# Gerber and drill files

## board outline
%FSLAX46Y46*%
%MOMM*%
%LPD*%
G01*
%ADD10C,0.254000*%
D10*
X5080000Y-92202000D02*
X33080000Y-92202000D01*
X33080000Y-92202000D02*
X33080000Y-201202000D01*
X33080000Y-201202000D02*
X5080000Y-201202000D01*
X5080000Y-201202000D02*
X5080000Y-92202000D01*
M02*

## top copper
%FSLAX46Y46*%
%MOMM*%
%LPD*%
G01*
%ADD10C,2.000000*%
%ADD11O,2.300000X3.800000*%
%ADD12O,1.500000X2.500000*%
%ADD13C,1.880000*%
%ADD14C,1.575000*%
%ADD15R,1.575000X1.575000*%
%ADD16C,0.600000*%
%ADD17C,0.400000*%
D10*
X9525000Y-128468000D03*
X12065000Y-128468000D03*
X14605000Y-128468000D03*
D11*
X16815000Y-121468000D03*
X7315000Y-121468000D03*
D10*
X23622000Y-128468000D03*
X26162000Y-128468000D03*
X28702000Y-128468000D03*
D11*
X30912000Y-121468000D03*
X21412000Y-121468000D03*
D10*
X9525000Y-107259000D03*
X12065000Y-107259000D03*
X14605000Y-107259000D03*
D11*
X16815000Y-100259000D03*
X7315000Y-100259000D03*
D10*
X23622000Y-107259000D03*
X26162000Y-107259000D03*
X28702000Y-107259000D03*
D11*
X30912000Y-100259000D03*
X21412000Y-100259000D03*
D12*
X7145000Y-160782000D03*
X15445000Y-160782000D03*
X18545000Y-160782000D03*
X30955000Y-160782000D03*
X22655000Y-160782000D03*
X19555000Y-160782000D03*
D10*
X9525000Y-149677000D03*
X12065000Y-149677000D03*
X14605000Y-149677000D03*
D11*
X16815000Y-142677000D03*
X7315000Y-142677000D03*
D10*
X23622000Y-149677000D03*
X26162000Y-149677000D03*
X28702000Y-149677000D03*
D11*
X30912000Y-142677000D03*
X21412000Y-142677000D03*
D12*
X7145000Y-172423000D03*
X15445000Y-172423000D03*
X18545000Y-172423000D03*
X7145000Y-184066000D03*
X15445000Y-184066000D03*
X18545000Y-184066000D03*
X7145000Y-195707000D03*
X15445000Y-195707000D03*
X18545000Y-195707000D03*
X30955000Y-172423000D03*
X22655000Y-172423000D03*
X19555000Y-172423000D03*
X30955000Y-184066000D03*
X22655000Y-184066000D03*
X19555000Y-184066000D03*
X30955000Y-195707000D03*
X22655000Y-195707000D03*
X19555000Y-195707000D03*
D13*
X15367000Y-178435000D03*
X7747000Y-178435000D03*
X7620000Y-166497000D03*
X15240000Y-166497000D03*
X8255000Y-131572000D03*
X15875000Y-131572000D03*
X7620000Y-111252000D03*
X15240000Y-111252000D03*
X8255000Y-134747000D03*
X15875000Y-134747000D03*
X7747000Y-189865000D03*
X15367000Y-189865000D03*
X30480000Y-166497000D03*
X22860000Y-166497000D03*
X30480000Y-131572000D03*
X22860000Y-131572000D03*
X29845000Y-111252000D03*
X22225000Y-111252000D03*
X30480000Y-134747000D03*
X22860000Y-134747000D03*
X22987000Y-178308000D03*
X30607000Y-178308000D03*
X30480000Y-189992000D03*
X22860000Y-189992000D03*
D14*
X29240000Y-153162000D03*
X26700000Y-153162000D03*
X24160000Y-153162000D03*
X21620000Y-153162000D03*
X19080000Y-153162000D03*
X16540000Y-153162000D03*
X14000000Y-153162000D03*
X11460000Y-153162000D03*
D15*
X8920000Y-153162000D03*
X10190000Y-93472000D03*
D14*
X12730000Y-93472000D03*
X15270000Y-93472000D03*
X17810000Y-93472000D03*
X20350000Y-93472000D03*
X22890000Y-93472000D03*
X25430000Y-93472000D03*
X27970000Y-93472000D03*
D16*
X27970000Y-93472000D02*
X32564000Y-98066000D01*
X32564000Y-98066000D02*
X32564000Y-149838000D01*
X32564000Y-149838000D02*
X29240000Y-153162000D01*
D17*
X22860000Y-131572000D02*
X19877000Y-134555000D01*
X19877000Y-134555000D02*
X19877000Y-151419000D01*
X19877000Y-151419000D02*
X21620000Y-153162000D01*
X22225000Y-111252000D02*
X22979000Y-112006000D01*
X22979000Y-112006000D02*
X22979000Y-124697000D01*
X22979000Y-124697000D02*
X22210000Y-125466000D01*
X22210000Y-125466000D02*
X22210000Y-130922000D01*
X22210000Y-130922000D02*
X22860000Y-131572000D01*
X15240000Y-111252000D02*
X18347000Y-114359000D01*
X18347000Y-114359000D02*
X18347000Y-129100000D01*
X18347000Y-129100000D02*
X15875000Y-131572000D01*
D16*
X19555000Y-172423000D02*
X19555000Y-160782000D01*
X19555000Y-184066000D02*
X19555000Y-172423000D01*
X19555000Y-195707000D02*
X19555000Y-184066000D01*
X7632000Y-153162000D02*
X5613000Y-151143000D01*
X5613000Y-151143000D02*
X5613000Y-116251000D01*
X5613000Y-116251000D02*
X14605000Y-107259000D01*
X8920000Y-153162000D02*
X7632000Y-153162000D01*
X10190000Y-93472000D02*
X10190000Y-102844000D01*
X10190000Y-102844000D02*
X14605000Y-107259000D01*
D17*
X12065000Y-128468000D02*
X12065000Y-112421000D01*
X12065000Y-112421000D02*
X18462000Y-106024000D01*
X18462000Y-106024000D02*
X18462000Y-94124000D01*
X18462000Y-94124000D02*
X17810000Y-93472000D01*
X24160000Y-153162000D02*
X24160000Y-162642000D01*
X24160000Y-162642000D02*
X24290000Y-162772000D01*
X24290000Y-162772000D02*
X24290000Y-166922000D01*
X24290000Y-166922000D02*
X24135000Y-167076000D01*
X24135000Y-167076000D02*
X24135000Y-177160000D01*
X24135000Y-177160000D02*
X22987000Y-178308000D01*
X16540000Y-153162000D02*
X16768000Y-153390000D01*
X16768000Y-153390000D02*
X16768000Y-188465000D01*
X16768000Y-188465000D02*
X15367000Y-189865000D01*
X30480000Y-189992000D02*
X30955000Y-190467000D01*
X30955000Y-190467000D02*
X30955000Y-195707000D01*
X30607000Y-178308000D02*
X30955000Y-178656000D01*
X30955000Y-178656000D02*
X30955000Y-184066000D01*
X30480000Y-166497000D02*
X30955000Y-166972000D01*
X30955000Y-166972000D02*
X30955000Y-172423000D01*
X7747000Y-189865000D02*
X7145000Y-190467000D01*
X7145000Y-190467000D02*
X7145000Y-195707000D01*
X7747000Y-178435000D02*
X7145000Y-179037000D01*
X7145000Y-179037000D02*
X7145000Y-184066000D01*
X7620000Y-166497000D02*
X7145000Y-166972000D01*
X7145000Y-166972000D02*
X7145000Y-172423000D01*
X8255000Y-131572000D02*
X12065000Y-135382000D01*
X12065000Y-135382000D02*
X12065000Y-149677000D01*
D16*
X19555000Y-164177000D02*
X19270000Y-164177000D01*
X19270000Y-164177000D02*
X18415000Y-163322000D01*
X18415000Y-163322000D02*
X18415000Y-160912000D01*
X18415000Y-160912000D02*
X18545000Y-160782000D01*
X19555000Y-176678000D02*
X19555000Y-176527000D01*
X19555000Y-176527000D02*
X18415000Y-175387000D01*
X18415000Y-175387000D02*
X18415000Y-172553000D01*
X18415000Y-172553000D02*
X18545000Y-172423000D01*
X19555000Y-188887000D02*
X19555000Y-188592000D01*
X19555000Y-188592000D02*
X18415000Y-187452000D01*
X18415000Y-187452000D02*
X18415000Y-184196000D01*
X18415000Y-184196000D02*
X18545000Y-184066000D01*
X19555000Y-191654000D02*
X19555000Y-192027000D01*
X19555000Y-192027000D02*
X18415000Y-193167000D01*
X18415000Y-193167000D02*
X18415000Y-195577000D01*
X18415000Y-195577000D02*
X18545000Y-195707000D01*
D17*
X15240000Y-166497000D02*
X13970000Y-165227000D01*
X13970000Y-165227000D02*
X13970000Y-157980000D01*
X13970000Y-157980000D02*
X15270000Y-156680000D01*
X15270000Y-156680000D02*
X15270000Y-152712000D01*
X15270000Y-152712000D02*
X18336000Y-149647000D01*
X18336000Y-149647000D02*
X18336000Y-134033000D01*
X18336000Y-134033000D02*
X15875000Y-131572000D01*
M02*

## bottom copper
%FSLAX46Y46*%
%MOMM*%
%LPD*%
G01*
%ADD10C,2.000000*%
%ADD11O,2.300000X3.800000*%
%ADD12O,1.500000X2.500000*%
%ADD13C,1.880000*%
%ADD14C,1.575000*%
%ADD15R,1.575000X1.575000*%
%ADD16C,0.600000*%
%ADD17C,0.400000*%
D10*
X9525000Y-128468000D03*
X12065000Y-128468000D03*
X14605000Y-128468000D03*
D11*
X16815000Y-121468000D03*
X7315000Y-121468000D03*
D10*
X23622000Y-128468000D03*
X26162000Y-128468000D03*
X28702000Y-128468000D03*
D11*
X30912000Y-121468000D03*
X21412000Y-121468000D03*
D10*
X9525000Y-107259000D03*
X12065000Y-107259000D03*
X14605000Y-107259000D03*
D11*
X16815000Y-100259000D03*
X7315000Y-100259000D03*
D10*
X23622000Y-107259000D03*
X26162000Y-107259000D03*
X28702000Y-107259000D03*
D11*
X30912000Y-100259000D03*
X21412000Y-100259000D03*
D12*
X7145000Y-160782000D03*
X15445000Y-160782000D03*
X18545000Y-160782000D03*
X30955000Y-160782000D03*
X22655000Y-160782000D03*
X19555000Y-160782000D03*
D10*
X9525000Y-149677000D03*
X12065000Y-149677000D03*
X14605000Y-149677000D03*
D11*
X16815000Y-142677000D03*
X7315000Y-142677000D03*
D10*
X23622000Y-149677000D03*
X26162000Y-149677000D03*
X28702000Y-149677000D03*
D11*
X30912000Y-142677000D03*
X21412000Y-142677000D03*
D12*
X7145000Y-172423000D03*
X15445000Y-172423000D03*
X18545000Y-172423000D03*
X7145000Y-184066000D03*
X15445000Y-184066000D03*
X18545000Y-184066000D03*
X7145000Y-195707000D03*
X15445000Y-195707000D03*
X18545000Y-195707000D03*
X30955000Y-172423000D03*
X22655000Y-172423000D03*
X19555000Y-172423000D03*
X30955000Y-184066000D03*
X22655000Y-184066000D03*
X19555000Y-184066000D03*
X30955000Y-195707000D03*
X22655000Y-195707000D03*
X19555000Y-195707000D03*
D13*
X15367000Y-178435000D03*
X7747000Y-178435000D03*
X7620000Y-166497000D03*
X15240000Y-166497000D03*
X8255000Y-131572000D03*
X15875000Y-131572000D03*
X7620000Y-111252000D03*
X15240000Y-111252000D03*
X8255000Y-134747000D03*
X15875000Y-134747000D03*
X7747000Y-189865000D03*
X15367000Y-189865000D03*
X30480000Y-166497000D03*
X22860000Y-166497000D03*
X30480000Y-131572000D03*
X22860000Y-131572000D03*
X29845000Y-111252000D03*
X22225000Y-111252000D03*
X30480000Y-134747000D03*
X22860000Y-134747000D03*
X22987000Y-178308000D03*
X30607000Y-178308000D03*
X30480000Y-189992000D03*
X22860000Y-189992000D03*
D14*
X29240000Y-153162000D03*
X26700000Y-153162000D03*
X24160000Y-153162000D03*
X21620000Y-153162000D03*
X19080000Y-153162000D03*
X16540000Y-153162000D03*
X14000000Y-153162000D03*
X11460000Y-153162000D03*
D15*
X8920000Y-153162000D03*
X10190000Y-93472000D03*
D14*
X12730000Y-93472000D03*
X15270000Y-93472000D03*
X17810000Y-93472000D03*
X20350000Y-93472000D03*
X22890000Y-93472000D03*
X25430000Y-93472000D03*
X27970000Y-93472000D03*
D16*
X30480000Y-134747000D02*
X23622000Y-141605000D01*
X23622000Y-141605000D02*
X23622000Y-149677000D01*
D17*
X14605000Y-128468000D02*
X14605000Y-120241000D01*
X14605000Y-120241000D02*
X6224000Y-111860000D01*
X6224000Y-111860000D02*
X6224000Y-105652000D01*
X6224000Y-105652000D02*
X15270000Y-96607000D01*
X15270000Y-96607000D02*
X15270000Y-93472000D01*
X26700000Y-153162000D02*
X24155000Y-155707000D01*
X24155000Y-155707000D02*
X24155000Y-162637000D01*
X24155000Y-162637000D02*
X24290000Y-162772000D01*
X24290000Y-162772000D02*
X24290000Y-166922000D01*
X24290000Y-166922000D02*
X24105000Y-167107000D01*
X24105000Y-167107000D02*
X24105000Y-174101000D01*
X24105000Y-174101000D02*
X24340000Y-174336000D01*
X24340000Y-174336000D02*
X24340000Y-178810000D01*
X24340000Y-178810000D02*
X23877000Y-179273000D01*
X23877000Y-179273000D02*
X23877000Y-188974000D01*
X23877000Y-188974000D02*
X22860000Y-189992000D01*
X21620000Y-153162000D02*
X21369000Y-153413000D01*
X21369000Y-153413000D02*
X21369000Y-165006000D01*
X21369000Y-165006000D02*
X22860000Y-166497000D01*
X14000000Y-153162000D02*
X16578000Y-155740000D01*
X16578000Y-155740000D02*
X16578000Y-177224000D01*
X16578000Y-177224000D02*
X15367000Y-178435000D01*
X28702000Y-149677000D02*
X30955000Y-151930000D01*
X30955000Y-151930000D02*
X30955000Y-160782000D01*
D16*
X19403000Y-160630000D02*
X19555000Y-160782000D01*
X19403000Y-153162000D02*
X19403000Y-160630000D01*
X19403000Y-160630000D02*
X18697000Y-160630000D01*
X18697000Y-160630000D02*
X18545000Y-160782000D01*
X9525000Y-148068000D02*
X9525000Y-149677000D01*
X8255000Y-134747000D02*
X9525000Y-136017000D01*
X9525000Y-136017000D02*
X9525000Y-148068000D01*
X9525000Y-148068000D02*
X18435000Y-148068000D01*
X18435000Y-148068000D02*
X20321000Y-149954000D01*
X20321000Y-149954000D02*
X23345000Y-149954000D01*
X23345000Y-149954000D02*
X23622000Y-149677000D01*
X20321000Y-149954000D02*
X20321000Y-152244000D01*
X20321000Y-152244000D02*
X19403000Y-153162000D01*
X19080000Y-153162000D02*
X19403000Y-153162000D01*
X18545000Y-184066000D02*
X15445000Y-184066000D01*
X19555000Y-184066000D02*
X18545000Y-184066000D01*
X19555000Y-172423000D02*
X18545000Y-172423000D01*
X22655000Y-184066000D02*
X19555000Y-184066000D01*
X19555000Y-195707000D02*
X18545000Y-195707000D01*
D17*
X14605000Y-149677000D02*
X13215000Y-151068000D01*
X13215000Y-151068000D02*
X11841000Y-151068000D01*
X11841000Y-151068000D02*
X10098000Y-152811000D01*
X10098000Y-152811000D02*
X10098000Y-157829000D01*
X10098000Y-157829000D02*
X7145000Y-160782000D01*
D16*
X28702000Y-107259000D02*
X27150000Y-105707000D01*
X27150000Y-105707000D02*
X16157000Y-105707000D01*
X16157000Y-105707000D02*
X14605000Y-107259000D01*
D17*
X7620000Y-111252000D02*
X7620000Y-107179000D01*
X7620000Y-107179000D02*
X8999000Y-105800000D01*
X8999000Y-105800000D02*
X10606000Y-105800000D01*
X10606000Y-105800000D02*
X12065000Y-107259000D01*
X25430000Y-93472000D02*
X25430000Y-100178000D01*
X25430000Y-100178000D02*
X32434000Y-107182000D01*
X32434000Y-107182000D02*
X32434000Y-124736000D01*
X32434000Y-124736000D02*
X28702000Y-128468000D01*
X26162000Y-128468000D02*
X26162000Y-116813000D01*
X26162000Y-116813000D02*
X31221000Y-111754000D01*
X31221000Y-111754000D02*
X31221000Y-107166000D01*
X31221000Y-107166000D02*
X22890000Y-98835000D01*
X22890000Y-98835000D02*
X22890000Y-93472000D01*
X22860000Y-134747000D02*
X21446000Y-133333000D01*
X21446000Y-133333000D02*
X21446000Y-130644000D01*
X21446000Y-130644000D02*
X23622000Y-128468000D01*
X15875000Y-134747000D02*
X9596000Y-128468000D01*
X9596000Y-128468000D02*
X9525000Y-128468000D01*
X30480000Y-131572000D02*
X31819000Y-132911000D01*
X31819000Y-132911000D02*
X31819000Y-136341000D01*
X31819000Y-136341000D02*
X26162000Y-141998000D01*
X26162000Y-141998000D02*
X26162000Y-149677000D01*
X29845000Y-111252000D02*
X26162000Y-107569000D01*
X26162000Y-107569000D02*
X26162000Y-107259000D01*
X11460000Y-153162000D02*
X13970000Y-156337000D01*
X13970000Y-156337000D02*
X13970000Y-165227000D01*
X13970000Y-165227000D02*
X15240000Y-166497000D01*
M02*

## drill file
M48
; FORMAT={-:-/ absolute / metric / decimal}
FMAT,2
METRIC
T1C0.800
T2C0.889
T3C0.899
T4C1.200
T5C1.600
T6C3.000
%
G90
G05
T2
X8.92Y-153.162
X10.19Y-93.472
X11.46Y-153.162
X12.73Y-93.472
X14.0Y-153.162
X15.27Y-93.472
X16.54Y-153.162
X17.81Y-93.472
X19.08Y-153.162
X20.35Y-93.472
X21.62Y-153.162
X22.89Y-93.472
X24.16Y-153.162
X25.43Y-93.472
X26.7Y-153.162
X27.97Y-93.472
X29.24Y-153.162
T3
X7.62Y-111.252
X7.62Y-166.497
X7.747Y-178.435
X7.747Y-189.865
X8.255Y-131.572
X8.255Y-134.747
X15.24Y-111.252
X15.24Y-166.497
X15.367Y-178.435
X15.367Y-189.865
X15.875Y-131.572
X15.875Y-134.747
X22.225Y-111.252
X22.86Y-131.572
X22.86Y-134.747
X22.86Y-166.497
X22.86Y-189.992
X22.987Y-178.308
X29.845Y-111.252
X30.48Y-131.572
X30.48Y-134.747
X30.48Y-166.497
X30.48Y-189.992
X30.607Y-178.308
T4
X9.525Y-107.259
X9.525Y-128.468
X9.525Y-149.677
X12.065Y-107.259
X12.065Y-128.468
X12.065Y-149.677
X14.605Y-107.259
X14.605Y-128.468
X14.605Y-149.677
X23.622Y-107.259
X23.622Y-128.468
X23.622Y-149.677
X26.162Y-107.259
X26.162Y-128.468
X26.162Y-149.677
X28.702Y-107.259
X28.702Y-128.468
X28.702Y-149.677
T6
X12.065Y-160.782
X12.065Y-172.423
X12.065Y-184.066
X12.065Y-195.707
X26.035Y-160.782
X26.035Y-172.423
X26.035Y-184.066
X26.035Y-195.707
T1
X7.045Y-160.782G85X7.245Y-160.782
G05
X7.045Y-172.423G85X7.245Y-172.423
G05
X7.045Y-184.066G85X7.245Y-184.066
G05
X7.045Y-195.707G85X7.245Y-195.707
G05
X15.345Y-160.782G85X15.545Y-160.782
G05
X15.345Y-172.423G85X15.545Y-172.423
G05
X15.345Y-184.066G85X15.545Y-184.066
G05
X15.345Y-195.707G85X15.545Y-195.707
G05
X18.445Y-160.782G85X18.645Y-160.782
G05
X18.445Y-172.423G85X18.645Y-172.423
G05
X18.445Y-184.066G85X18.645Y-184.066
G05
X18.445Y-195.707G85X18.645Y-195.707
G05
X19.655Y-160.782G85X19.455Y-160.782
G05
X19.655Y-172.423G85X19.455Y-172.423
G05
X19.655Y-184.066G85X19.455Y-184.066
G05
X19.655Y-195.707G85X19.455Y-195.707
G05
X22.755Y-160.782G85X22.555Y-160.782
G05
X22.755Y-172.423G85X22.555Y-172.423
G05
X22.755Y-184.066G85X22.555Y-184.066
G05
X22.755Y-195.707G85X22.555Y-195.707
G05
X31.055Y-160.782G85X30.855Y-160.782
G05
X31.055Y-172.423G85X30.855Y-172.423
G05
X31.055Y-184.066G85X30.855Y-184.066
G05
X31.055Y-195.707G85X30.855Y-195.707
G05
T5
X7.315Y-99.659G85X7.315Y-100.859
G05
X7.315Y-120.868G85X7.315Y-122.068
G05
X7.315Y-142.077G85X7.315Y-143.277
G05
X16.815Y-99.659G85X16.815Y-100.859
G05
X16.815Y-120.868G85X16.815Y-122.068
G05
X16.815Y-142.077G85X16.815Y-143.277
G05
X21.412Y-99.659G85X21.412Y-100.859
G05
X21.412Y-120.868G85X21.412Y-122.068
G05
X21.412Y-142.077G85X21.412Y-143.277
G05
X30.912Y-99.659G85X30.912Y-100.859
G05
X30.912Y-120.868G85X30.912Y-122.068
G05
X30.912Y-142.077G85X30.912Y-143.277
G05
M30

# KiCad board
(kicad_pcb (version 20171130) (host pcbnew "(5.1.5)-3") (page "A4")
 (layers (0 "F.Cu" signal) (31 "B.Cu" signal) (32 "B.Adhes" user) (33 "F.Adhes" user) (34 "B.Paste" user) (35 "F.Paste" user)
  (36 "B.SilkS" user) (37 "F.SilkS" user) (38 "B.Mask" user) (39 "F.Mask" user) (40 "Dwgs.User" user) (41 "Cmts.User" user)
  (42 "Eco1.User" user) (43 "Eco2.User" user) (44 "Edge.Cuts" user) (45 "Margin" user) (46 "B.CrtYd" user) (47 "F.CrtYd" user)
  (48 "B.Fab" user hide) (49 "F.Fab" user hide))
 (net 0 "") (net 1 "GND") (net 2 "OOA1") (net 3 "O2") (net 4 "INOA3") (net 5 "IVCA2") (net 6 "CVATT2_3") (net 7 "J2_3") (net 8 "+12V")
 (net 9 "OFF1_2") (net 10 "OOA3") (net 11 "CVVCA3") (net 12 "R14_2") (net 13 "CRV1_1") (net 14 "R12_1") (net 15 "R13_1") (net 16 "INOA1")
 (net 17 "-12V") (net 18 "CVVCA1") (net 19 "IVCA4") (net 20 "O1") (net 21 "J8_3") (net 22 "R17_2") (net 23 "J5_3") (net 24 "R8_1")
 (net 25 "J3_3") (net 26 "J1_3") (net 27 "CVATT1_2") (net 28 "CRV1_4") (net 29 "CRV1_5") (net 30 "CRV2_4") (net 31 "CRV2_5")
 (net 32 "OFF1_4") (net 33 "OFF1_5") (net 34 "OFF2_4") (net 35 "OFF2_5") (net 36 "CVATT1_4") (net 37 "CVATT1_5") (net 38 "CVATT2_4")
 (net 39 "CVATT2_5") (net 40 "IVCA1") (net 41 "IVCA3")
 (segment (start 30.48 134.747) (end 23.622 141.605) (width 0.6) (layer "B.Cu") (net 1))
 (segment (start 23.622 141.605) (end 23.622 149.677) (width 0.6) (layer "B.Cu") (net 1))
 (segment (start 14.605 128.468) (end 14.605 120.241) (width 0.4) (layer "B.Cu") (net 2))
 (segment (start 14.605 120.241) (end 6.224 111.86) (width 0.4) (layer "B.Cu") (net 2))
 (segment (start 6.224 111.86) (end 6.224 105.652) (width 0.4) (layer "B.Cu") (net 2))
 (segment (start 6.224 105.652) (end 15.27 96.607) (width 0.4) (layer "B.Cu") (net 2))
 (segment (start 15.27 96.607) (end 15.27 93.472) (width 0.4) (layer "B.Cu") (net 2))
 (segment (start 26.7 153.162) (end 24.155 155.707) (width 0.4) (layer "B.Cu") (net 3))
 (segment (start 24.155 155.707) (end 24.155 162.637) (width 0.4) (layer "B.Cu") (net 3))
 (segment (start 24.155 162.637) (end 24.29 162.772) (width 0.4) (layer "B.Cu") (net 3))
 (segment (start 24.29 162.772) (end 24.29 166.922) (width 0.4) (layer "B.Cu") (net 3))
 (segment (start 24.29 166.922) (end 24.105 167.107) (width 0.4) (layer "B.Cu") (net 3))
 (segment (start 24.105 167.107) (end 24.105 174.101) (width 0.4) (layer "B.Cu") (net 3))
 (segment (start 24.105 174.101) (end 24.34 174.336) (width 0.4) (layer "B.Cu") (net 3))
 (segment (start 24.34 174.336) (end 24.34 178.81) (width 0.4) (layer "B.Cu") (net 3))
 (segment (start 24.34 178.81) (end 23.877 179.273) (width 0.4) (layer "B.Cu") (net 3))
 (segment (start 23.877 179.273) (end 23.877 188.974) (width 0.4) (layer "B.Cu") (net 3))
 (segment (start 23.877 188.974) (end 22.86 189.992) (width 0.4) (layer "B.Cu") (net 3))
 (segment (start 21.62 153.162) (end 21.369 153.413) (width 0.4) (layer "B.Cu") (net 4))
 (segment (start 21.369 153.413) (end 21.369 165.006) (width 0.4) (layer "B.Cu") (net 4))
 (segment (start 21.369 165.006) (end 22.86 166.497) (width 0.4) (layer "B.Cu") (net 4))
 (segment (start 14 153.162) (end 16.578 155.74) (width 0.4) (layer "B.Cu") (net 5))
 (segment (start 16.578 155.74) (end 16.578 177.224) (width 0.4) (layer "B.Cu") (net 5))
 (segment (start 16.578 177.224) (end 15.367 178.435) (width 0.4) (layer "B.Cu") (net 5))
 (segment (start 28.702 149.677) (end 30.955 151.93) (width 0.4) (layer "B.Cu") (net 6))
 (segment (start 30.955 151.93) (end 30.955 160.782) (width 0.4) (layer "B.Cu") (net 6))
 (segment (start 19.403 160.63) (end 19.555 160.782) (width 0.6) (layer "B.Cu") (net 1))
 (segment (start 19.403 153.162) (end 19.403 160.63) (width 0.6) (layer "B.Cu") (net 1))
 (segment (start 19.403 160.63) (end 18.697 160.63) (width 0.6) (layer "B.Cu") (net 1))
 (segment (start 18.697 160.63) (end 18.545 160.782) (width 0.6) (layer "B.Cu") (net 1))
 (segment (start 9.525 148.068) (end 9.525 149.677) (width 0.6) (layer "B.Cu") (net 1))
 (segment (start 8.255 134.747) (end 9.525 136.017) (width 0.6) (layer "B.Cu") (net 1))
 (segment (start 9.525 136.017) (end 9.525 148.068) (width 0.6) (layer "B.Cu") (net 1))
 (segment (start 9.525 148.068) (end 18.435 148.068) (width 0.6) (layer "B.Cu") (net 1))
 (segment (start 18.435 148.068) (end 20.321 149.954) (width 0.6) (layer "B.Cu") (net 1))
 (segment (start 20.321 149.954) (end 23.345 149.954) (width 0.6) (layer "B.Cu") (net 1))
 (segment (start 23.345 149.954) (end 23.622 149.677) (width 0.6) (layer "B.Cu") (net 1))
 (segment (start 20.321 149.954) (end 20.321 152.244) (width 0.6) (layer "B.Cu") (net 1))
 (segment (start 20.321 152.244) (end 19.403 153.162) (width 0.6) (layer "B.Cu") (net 1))
 (segment (start 19.08 153.162) (end 19.403 153.162) (width 0.6) (layer "B.Cu") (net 1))
 (segment (start 18.545 184.066) (end 15.445 184.066) (width 0.6) (layer "B.Cu") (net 1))
 (segment (start 19.555 184.066) (end 18.545 184.066) (width 0.6) (layer "B.Cu") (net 1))
 (segment (start 19.555 172.423) (end 18.545 172.423) (width 0.6) (layer "B.Cu") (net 1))
 (segment (start 22.655 184.066) (end 19.555 184.066) (width 0.6) (layer "B.Cu") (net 1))
 (segment (start 19.555 195.707) (end 18.545 195.707) (width 0.6) (layer "B.Cu") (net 1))
 (segment (start 14.605 149.677) (end 13.215 151.068) (width 0.4) (layer "B.Cu") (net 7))
 (segment (start 13.215 151.068) (end 11.841 151.068) (width 0.4) (layer "B.Cu") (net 7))
 (segment (start 11.841 151.068) (end 10.098 152.811) (width 0.4) (layer "B.Cu") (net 7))
 (segment (start 10.098 152.811) (end 10.098 157.829) (width 0.4) (layer "B.Cu") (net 7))
 (segment (start 10.098 157.829) (end 7.145 160.782) (width 0.4) (layer "B.Cu") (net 7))
 (segment (start 28.702 107.259) (end 27.15 105.707) (width 0.6) (layer "B.Cu") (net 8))
 (segment (start 27.15 105.707) (end 16.157 105.707) (width 0.6) (layer "B.Cu") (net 8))
 (segment (start 16.157 105.707) (end 14.605 107.259) (width 0.6) (layer "B.Cu") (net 8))
 (segment (start 7.62 111.252) (end 7.62 107.179) (width 0.4) (layer "B.Cu") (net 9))
 (segment (start 7.62 107.179) (end 8.999 105.8) (width 0.4) (layer "B.Cu") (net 9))
 (segment (start 8.999 105.8) (end 10.606 105.8) (width 0.4) (layer "B.Cu") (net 9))
 (segment (start 10.606 105.8) (end 12.065 107.259) (width 0.4) (layer "B.Cu") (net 9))
 (segment (start 25.43 93.472) (end 25.43 100.178) (width 0.4) (layer "B.Cu") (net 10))
 (segment (start 25.43 100.178) (end 32.434 107.182) (width 0.4) (layer "B.Cu") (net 10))
 (segment (start 32.434 107.182) (end 32.434 124.736) (width 0.4) (layer "B.Cu") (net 10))
 (segment (start 32.434 124.736) (end 28.702 128.468) (width 0.4) (layer "B.Cu") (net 10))
 (segment (start 26.162 128.468) (end 26.162 116.813) (width 0.4) (layer "B.Cu") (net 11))
 (segment (start 26.162 116.813) (end 31.221 111.754) (width 0.4) (layer "B.Cu") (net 11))
 (segment (start 31.221 111.754) (end 31.221 107.166) (width 0.4) (layer "B.Cu") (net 11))
 (segment (start 31.221 107.166) (end 22.89 98.835) (width 0.4) (layer "B.Cu") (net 11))
 (segment (start 22.89 98.835) (end 22.89 93.472) (width 0.4) (layer "B.Cu") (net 11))
 (segment (start 22.86 134.747) (end 21.446 133.333) (width 0.4) (layer "B.Cu") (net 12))
 (segment (start 21.446 133.333) (end 21.446 130.644) (width 0.4) (layer "B.Cu") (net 12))
 (segment (start 21.446 130.644) (end 23.622 128.468) (width 0.4) (layer "B.Cu") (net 12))
 (segment (start 15.875 134.747) (end 9.596 128.468) (width 0.4) (layer "B.Cu") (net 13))
 (segment (start 9.596 128.468) (end 9.525 128.468) (width 0.4) (layer "B.Cu") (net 13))
 (segment (start 30.48 131.572) (end 31.819 132.911) (width 0.4) (layer "B.Cu") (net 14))
 (segment (start 31.819 132.911) (end 31.819 136.341) (width 0.4) (layer "B.Cu") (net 14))
 (segment (start 31.819 136.341) (end 26.162 141.998) (width 0.4) (layer "B.Cu") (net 14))
 (segment (start 26.162 141.998) (end 26.162 149.677) (width 0.4) (layer "B.Cu") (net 14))
 (segment (start 29.845 111.252) (end 26.162 107.569) (width 0.4) (layer "B.Cu") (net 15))
 (segment (start 26.162 107.569) (end 26.162 107.259) (width 0.4) (layer "B.Cu") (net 15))
 (segment (start 11.46 153.162) (end 13.97 156.337) (width 0.4) (layer "B.Cu") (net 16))
 (segment (start 13.97 156.337) (end 13.97 165.227) (width 0.4) (layer "B.Cu") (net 16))
 (segment (start 13.97 165.227) (end 15.24 166.497) (width 0.4) (layer "B.Cu") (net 16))
 (gr_line (start 5.08 92.202) (end 33.08 92.202) (width 0.254) (layer "Edge.Cuts"))
 (gr_line (start 33.08 92.202) (end 33.08 201.202) (width 0.254) (layer "Edge.Cuts"))
 (gr_line (start 33.08 201.202) (end 5.08 201.202) (width 0.254) (layer "Edge.Cuts"))
 (gr_line (start 5.08 201.202) (end 5.08 92.202) (width 0.254) (layer "Edge.Cuts"))
 (segment (start 27.97 93.472) (end 32.564 98.066) (width 0.6) (layer "F.Cu") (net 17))
 (segment (start 32.564 98.066) (end 32.564 149.838) (width 0.6) (layer "F.Cu") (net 17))
 (segment (start 32.564 149.838) (end 29.24 153.162) (width 0.6) (layer "F.Cu") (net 17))
 (segment (start 22.86 131.572) (end 19.877 134.555) (width 0.4) (layer "F.Cu") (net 4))
 (segment (start 19.877 134.555) (end 19.877 151.419) (width 0.4) (layer "F.Cu") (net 4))
 (segment (start 19.877 151.419) (end 21.62 153.162) (width 0.4) (layer "F.Cu") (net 4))
 (segment (start 22.225 111.252) (end 22.979 112.006) (width 0.4) (layer "F.Cu") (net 4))
 (segment (start 22.979 112.006) (end 22.979 124.697) (width 0.4) (layer "F.Cu") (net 4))
 (segment (start 22.979 124.697) (end 22.21 125.466) (width 0.4) (layer "F.Cu") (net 4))
 (segment (start 22.21 125.466) (end 22.21 130.922) (width 0.4) (layer "F.Cu") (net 4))
 (segment (start 22.21 130.922) (end 22.86 131.572) (width 0.4) (layer "F.Cu") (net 4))
 (segment (start 15.24 111.252) (end 18.347 114.359) (width 0.4) (layer "F.Cu") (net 16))
 (segment (start 18.347 114.359) (end 18.347 129.1) (width 0.4) (layer "F.Cu") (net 16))
 (segment (start 18.347 129.1) (end 15.875 131.572) (width 0.4) (layer "F.Cu") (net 16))
 (segment (start 19.555 172.423) (end 19.555 160.782) (width 0.6) (layer "F.Cu") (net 1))
 (segment (start 19.555 184.066) (end 19.555 172.423) (width 0.6) (layer "F.Cu") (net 1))
 (segment (start 19.555 195.707) (end 19.555 184.066) (width 0.6) (layer "F.Cu") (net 1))
 (segment (start 7.632 153.162) (end 5.613 151.143) (width 0.6) (layer "F.Cu") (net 8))
 (segment (start 5.613 151.143) (end 5.613 116.251) (width 0.6) (layer "F.Cu") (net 8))
 (segment (start 5.613 116.251) (end 14.605 107.259) (width 0.6) (layer "F.Cu") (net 8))
 (segment (start 8.92 153.162) (end 7.632 153.162) (width 0.6) (layer "F.Cu") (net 8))
 (segment (start 10.19 93.472) (end 10.19 102.844) (width 0.6) (layer "F.Cu") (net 8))
 (segment (start 10.19 102.844) (end 14.605 107.259) (width 0.6) (layer "F.Cu") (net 8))
 (segment (start 12.065 128.468) (end 12.065 112.421) (width 0.4) (layer "F.Cu") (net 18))
 (segment (start 12.065 112.421) (end 18.462 106.024) (width 0.4) (layer "F.Cu") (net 18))
 (segment (start 18.462 106.024) (end 18.462 94.124) (width 0.4) (layer "F.Cu") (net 18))
 (segment (start 18.462 94.124) (end 17.81 93.472) (width 0.4) (layer "F.Cu") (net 18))
 (segment (start 24.16 153.162) (end 24.16 162.642) (width 0.4) (layer "F.Cu") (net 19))
 (segment (start 24.16 162.642) (end 24.29 162.772) (width 0.4) (layer "F.Cu") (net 19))
 (segment (start 24.29 162.772) (end 24.29 166.922) (width 0.4) (layer "F.Cu") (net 19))
 (segment (start 24.29 166.922) (end 24.135 167.076) (width 0.4) (layer "F.Cu") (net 19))
 (segment (start 24.135 167.076) (end 24.135 177.16) (width 0.4) (layer "F.Cu") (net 19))
 (segment (start 24.135 177.16) (end 22.987 178.308) (width 0.4) (layer "F.Cu") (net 19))
 (segment (start 16.54 153.162) (end 16.768 153.39) (width 0.4) (layer "F.Cu") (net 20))
 (segment (start 16.768 153.39) (end 16.768 188.465) (width 0.4) (layer "F.Cu") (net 20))
 (segment (start 16.768 188.465) (end 15.367 189.865) (width 0.4) (layer "F.Cu") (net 20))
 (segment (start 30.48 189.992) (end 30.955 190.467) (width 0.4) (layer "F.Cu") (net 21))
 (segment (start 30.955 190.467) (end 30.955 195.707) (width 0.4) (layer "F.Cu") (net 21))
 (segment (start 30.607 178.308) (end 30.955 178.656) (width 0.4) (layer "F.Cu") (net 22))
 (segment (start 30.955 178.656) (end 30.955 184.066) (width 0.4) (layer "F.Cu") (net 22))
 (segment (start 30.48 166.497) (end 30.955 166.972) (width 0.4) (layer "F.Cu") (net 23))
 (segment (start 30.955 166.972) (end 30.955 172.423) (width 0.4) (layer "F.Cu") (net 23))
 (segment (start 7.747 189.865) (end 7.145 190.467) (width 0.4) (layer "F.Cu") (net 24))
 (segment (start 7.145 190.467) (end 7.145 195.707) (width 0.4) (layer "F.Cu") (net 24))
 (segment (start 7.747 178.435) (end 7.145 179.037) (width 0.4) (layer "F.Cu") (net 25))
 (segment (start 7.145 179.037) (end 7.145 184.066) (width 0.4) (layer "F.Cu") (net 25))
 (segment (start 7.62 166.497) (end 7.145 166.972) (width 0.4) (layer "F.Cu") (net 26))
 (segment (start 7.145 166.972) (end 7.145 172.423) (width 0.4) (layer "F.Cu") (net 26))
 (segment (start 8.255 131.572) (end 12.065 135.382) (width 0.4) (layer "F.Cu") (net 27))
 (segment (start 12.065 135.382) (end 12.065 149.677) (width 0.4) (layer "F.Cu") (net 27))
 (segment (start 19.555 164.177) (end 19.27 164.177) (width 0.6) (layer "F.Cu") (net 1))
 (segment (start 19.27 164.177) (end 18.415 163.322) (width 0.6) (layer "F.Cu") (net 1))
 (segment (start 18.415 163.322) (end 18.415 160.912) (width 0.6) (layer "F.Cu") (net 1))
 (segment (start 18.415 160.912) (end 18.545 160.782) (width 0.6) (layer "F.Cu") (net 1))
 (segment (start 19.555 176.678) (end 19.555 176.527) (width 0.6) (layer "F.Cu") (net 1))
 (segment (start 19.555 176.527) (end 18.415 175.387) (width 0.6) (layer "F.Cu") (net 1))
 (segment (start 18.415 175.387) (end 18.415 172.553) (width 0.6) (layer "F.Cu") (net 1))
 (segment (start 18.415 172.553) (end 18.545 172.423) (width 0.6) (layer "F.Cu") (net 1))
 (segment (start 19.555 188.887) (end 19.555 188.592) (width 0.6) (layer "F.Cu") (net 1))
 (segment (start 19.555 188.592) (end 18.415 187.452) (width 0.6) (layer "F.Cu") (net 1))
 (segment (start 18.415 187.452) (end 18.415 184.196) (width 0.6) (layer "F.Cu") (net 1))
 (segment (start 18.415 184.196) (end 18.545 184.066) (width 0.6) (layer "F.Cu") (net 1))
 (segment (start 19.555 191.654) (end 19.555 192.027) (width 0.6) (layer "F.Cu") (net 1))
 (segment (start 19.555 192.027) (end 18.415 193.167) (width 0.6) (layer "F.Cu") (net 1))
 (segment (start 18.415 193.167) (end 18.415 195.577) (width 0.6) (layer "F.Cu") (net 1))
 (segment (start 18.415 195.577) (end 18.545 195.707) (width 0.6) (layer "F.Cu") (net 1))
 (segment (start 15.24 166.497) (end 13.97 165.227) (width 0.4) (layer "F.Cu") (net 16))
 (segment (start 13.97 165.227) (end 13.97 157.98) (width 0.4) (layer "F.Cu") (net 16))
 (segment (start 13.97 157.98) (end 15.27 156.68) (width 0.4) (layer "F.Cu") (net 16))
 (segment (start 15.27 156.68) (end 15.27 152.712) (width 0.4) (layer "F.Cu") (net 16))
 (segment (start 15.27 152.712) (end 18.336 149.647) (width 0.4) (layer "F.Cu") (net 16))
 (segment (start 18.336 149.647) (end 18.336 134.033) (width 0.4) (layer "F.Cu") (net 16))
 (segment (start 18.336 134.033) (end 15.875 131.572) (width 0.4) (layer "F.Cu") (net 16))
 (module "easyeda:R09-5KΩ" (layer "F.Cu") (at 12.065 124.968)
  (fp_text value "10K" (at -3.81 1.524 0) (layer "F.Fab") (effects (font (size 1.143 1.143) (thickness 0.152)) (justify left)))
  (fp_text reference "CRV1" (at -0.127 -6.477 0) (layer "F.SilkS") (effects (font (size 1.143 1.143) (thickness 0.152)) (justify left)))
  (pad 1 thru_hole circle (at -2.54 3.5 0) (size 2 2) (layers "*.Cu" "*.Paste" "*.Mask") (drill 1.2) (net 13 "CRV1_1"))
  (pad 2 thru_hole circle (at 0 3.5 0) (size 2 2) (layers "*.Cu" "*.Paste" "*.Mask") (drill 1.2) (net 18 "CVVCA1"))
  (pad 3 thru_hole circle (at 2.54 3.5 0) (size 2 2) (layers "*.Cu" "*.Paste" "*.Mask") (drill 1.2) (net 2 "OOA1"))
  (pad 4 thru_hole oval (at 4.75 -3.5 0) (size 2.3 3.8) (layers "*.Cu" "*.Paste" "*.Mask") (drill oval 1.6 2.8) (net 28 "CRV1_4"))
  (pad 5 thru_hole oval (at -4.75 -3.5 0) (size 2.3 3.8) (layers "*.Cu" "*.Paste" "*.Mask") (drill oval 1.6 2.8) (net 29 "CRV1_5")))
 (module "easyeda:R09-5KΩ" (layer "F.Cu") (at 26.162 124.968)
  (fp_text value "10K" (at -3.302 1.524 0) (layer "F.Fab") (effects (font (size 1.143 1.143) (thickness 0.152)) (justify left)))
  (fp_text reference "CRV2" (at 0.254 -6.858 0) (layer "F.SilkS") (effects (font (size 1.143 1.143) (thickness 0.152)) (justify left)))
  (pad 1 thru_hole circle (at -2.54 3.5 0) (size 2 2) (layers "*.Cu" "*.Paste" "*.Mask") (drill 1.2) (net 12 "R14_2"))
  (pad 2 thru_hole circle (at 0 3.5 0) (size 2 2) (layers "*.Cu" "*.Paste" "*.Mask") (drill 1.2) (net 11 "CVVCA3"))
  (pad 3 thru_hole circle (at 2.54 3.5 0) (size 2 2) (layers "*.Cu" "*.Paste" "*.Mask") (drill 1.2) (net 10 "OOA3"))
  (pad 4 thru_hole oval (at 4.75 -3.5 0) (size 2.3 3.8) (layers "*.Cu" "*.Paste" "*.Mask") (drill oval 1.6 2.8) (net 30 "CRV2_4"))
  (pad 5 thru_hole oval (at -4.75 -3.5 0) (size 2.3 3.8) (layers "*.Cu" "*.Paste" "*.Mask") (drill oval 1.6 2.8) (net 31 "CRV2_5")))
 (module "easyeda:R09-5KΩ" (layer "F.Cu") (at 12.065 103.759)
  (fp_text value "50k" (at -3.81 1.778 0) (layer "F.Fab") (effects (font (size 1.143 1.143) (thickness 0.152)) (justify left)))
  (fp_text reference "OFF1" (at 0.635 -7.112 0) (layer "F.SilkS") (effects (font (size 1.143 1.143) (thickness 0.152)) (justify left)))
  (pad 1 thru_hole circle (at -2.54 3.5 0) (size 2 2) (layers "*.Cu" "*.Paste" "*.Mask") (drill 1.2))
  (pad 2 thru_hole circle (at 0 3.5 0) (size 2 2) (layers "*.Cu" "*.Paste" "*.Mask") (drill 1.2) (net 9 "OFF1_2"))
  (pad 3 thru_hole circle (at 2.54 3.5 0) (size 2 2) (layers "*.Cu" "*.Paste" "*.Mask") (drill 1.2) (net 8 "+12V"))
  (pad 4 thru_hole oval (at 4.75 -3.5 0) (size 2.3 3.8) (layers "*.Cu" "*.Paste" "*.Mask") (drill oval 1.6 2.8) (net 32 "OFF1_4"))
  (pad 5 thru_hole oval (at -4.75 -3.5 0) (size 2.3 3.8) (layers "*.Cu" "*.Paste" "*.Mask") (drill oval 1.6 2.8) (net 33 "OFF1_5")))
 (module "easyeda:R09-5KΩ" (layer "F.Cu") (at 26.162 103.759)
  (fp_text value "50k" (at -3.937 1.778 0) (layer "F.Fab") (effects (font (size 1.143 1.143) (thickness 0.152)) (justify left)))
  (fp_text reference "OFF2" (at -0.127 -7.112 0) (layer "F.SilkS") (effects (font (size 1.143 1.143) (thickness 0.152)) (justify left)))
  (pad 1 thru_hole circle (at -2.54 3.5 0) (size 2 2) (layers "*.Cu" "*.Paste" "*.Mask") (drill 1.2))
  (pad 2 thru_hole circle (at 0 3.5 0) (size 2 2) (layers "*.Cu" "*.Paste" "*.Mask") (drill 1.2) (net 15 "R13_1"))
  (pad 3 thru_hole circle (at 2.54 3.5 0) (size 2 2) (layers "*.Cu" "*.Paste" "*.Mask") (drill 1.2) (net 8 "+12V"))
  (pad 4 thru_hole oval (at 4.75 -3.5 0) (size 2.3 3.8) (layers "*.Cu" "*.Paste" "*.Mask") (drill oval 1.6 2.8) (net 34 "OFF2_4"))
  (pad 5 thru_hole oval (at -4.75 -3.5 0) (size 2.3 3.8) (layers "*.Cu" "*.Paste" "*.Mask") (drill oval 1.6 2.8) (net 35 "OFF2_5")))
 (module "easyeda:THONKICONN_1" (layer "F.Cu") (at 12.065 160.782 90)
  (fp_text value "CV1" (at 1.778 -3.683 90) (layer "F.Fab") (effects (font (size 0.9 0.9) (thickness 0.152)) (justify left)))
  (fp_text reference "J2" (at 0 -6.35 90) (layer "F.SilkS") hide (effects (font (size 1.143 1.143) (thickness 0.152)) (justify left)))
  (pad "" np_thru_hole circle (at 0 0) (size 3 3) (drill 3) (layers "*.Cu" "*.Mask"))
  (pad 3 thru_hole oval (at 0 -4.92 90) (size 2.5 1.5) (layers "*.Cu" "*.Paste" "*.Mask") (drill oval 0.8 1) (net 7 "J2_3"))
  (pad 2 thru_hole oval (at 0 3.38 90) (size 2.5 1.5) (layers "*.Cu" "*.Paste" "*.Mask") (drill oval 0.8 1))
  (pad 1 thru_hole oval (at 0 6.48 90) (size 2.5 1.5) (layers "*.Cu" "*.Paste" "*.Mask") (drill oval 0.8 1) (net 1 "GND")))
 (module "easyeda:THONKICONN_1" (layer "F.Cu") (at 26.035 160.782 -90)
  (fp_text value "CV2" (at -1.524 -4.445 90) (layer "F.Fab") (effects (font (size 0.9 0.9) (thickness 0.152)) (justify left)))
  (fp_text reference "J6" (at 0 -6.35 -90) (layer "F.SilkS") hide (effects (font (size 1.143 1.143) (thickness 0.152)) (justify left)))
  (pad "" np_thru_hole circle (at 0 0) (size 3 3) (drill 3) (layers "*.Cu" "*.Mask"))
  (pad 3 thru_hole oval (at 0 -4.92 -90) (size 2.5 1.5) (layers "*.Cu" "*.Paste" "*.Mask") (drill oval 0.8 1) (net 6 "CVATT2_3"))
  (pad 2 thru_hole oval (at 0 3.38 -90) (size 2.5 1.5) (layers "*.Cu" "*.Paste" "*.Mask") (drill oval 0.8 1))
  (pad 1 thru_hole oval (at 0 6.48 -90) (size 2.5 1.5) (layers "*.Cu" "*.Paste" "*.Mask") (drill oval 0.8 1) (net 1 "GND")))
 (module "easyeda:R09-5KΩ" (layer "F.Cu") (at 12.065 146.177)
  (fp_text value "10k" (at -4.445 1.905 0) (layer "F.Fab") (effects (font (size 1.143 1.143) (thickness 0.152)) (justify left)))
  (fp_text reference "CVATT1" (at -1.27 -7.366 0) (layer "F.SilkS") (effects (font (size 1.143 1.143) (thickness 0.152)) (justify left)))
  (pad 1 thru_hole circle (at -2.54 3.5 0) (size 2 2) (layers "*.Cu" "*.Paste" "*.Mask") (drill 1.2) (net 1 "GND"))
  (pad 2 thru_hole circle (at 0 3.5 0) (size 2 2) (layers "*.Cu" "*.Paste" "*.Mask") (drill 1.2) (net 27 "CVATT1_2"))
  (pad 3 thru_hole circle (at 2.54 3.5 0) (size 2 2) (layers "*.Cu" "*.Paste" "*.Mask") (drill 1.2) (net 7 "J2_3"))
  (pad 4 thru_hole oval (at 4.75 -3.5 0) (size 2.3 3.8) (layers "*.Cu" "*.Paste" "*.Mask") (drill oval 1.6 2.8) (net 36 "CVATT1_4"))
  (pad 5 thru_hole oval (at -4.75 -3.5 0) (size 2.3 3.8) (layers "*.Cu" "*.Paste" "*.Mask") (drill oval 1.6 2.8) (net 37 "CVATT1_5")))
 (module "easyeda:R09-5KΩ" (layer "F.Cu") (at 26.162 146.177)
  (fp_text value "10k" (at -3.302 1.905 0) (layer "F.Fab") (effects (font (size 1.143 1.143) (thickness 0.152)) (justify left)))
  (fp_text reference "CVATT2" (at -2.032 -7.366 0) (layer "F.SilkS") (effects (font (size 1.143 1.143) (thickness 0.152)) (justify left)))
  (pad 1 thru_hole circle (at -2.54 3.5 0) (size 2 2) (layers "*.Cu" "*.Paste" "*.Mask") (drill 1.2) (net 1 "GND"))
  (pad 2 thru_hole circle (at 0 3.5 0) (size 2 2) (layers "*.Cu" "*.Paste" "*.Mask") (drill 1.2) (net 14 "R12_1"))
  (pad 3 thru_hole circle (at 2.54 3.5 0) (size 2 2) (layers "*.Cu" "*.Paste" "*.Mask") (drill 1.2) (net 6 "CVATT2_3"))
  (pad 4 thru_hole oval (at 4.75 -3.5 0) (size 2.3 3.8) (layers "*.Cu" "*.Paste" "*.Mask") (drill oval 1.6 2.8) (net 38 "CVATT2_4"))
  (pad 5 thru_hole oval (at -4.75 -3.5 0) (size 2.3 3.8) (layers "*.Cu" "*.Paste" "*.Mask") (drill oval 1.6 2.8) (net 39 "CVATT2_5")))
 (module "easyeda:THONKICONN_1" (layer "F.Cu") (at 12.065 172.423 90)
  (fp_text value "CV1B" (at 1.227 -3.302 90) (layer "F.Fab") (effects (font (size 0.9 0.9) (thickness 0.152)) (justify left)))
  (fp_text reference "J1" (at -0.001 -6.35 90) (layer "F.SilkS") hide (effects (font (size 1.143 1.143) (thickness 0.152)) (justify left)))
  (pad "" np_thru_hole circle (at 0 0) (size 3 3) (drill 3) (layers "*.Cu" "*.Mask"))
  (pad 3 thru_hole oval (at 0 -4.92 90) (size 2.5 1.5) (layers "*.Cu" "*.Paste" "*.Mask") (drill oval 0.8 1) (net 26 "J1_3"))
  (pad 2 thru_hole oval (at 0 3.38 90) (size 2.5 1.5) (layers "*.Cu" "*.Paste" "*.Mask") (drill oval 0.8 1))
  (pad 1 thru_hole oval (at 0 6.48 90) (size 2.5 1.5) (layers "*.Cu" "*.Paste" "*.Mask") (drill oval 0.8 1) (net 1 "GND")))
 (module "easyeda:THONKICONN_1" (layer "F.Cu") (at 12.065 184.066 90)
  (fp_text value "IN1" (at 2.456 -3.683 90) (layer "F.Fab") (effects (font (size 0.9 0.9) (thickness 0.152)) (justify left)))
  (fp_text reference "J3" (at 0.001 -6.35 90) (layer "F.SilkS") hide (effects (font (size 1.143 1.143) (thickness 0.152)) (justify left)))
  (pad "" np_thru_hole circle (at 0 0) (size 3 3) (drill 3) (layers "*.Cu" "*.Mask"))
  (pad 3 thru_hole oval (at 0 -4.92 90) (size 2.5 1.5) (layers "*.Cu" "*.Paste" "*.Mask") (drill oval 0.8 1) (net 25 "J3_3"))
  (pad 2 thru_hole oval (at 0 3.38 90) (size 2.5 1.5) (layers "*.Cu" "*.Paste" "*.Mask") (drill oval 0.8 1) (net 1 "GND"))
  (pad 1 thru_hole oval (at 0 6.48 90) (size 2.5 1.5) (layers "*.Cu" "*.Paste" "*.Mask") (drill oval 0.8 1) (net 1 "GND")))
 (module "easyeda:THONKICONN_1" (layer "F.Cu") (at 12.065 195.707 90)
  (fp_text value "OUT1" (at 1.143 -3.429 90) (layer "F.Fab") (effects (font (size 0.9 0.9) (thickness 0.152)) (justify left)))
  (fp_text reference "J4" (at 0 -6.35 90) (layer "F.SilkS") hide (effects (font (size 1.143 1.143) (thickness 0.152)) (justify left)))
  (pad "" np_thru_hole circle (at 0 0) (size 3 3) (drill 3) (layers "*.Cu" "*.Mask"))
  (pad 3 thru_hole oval (at 0 -4.92 90) (size 2.5 1.5) (layers "*.Cu" "*.Paste" "*.Mask") (drill oval 0.8 1) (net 24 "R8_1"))
  (pad 2 thru_hole oval (at 0 3.38 90) (size 2.5 1.5) (layers "*.Cu" "*.Paste" "*.Mask") (drill oval 0.8 1))
  (pad 1 thru_hole oval (at 0 6.48 90) (size 2.5 1.5) (layers "*.Cu" "*.Paste" "*.Mask") (drill oval 0.8 1) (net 1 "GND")))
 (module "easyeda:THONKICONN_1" (layer "F.Cu") (at 26.035 172.423 -90)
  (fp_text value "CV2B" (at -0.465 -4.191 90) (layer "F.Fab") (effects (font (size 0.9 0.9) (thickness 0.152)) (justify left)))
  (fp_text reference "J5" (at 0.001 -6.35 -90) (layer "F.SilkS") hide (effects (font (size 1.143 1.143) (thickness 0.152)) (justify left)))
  (pad "" np_thru_hole circle (at 0 0) (size 3 3) (drill 3) (layers "*.Cu" "*.Mask"))
  (pad 3 thru_hole oval (at 0 -4.92 -90) (size 2.5 1.5) (layers "*.Cu" "*.Paste" "*.Mask") (drill oval 0.8 1) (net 23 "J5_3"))
  (pad 2 thru_hole oval (at 0 3.38 -90) (size 2.5 1.5) (layers "*.Cu" "*.Paste" "*.Mask") (drill oval 0.8 1))
  (pad 1 thru_hole oval (at 0 6.48 -90) (size 2.5 1.5) (layers "*.Cu" "*.Paste" "*.Mask") (drill oval 0.8 1) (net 1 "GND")))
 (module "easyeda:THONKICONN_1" (layer "F.Cu") (at 26.035 184.066 -90)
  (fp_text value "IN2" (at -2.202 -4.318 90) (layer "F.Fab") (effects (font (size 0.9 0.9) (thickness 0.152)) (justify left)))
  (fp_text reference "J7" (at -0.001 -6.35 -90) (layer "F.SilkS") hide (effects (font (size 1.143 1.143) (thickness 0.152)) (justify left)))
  (pad "" np_thru_hole circle (at 0 0) (size 3 3) (drill 3) (layers "*.Cu" "*.Mask"))
  (pad 3 thru_hole oval (at 0 -4.92 -90) (size 2.5 1.5) (layers "*.Cu" "*.Paste" "*.Mask") (drill oval 0.8 1) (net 22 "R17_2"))
  (pad 2 thru_hole oval (at 0 3.38 -90) (size 2.5 1.5) (layers "*.Cu" "*.Paste" "*.Mask") (drill oval 0.8 1) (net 1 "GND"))
  (pad 1 thru_hole oval (at 0 6.48 -90) (size 2.5 1.5) (layers "*.Cu" "*.Paste" "*.Mask") (drill oval 0.8 1) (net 1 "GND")))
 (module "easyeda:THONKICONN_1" (layer "F.Cu") (at 26.035 195.707 -90)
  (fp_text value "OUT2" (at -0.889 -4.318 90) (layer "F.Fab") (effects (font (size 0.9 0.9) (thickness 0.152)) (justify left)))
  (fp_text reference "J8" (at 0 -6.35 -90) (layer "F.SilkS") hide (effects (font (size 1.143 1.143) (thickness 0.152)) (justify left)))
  (pad "" np_thru_hole circle (at 0 0) (size 3 3) (drill 3) (layers "*.Cu" "*.Mask"))
  (pad 3 thru_hole oval (at 0 -4.92 -90) (size 2.5 1.5) (layers "*.Cu" "*.Paste" "*.Mask") (drill oval 0.8 1) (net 21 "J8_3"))
  (pad 2 thru_hole oval (at 0 3.38 -90) (size 2.5 1.5) (layers "*.Cu" "*.Paste" "*.Mask") (drill oval 0.8 1))
  (pad 1 thru_hole oval (at 0 6.48 -90) (size 2.5 1.5) (layers "*.Cu" "*.Paste" "*.Mask") (drill oval 0.8 1) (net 1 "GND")))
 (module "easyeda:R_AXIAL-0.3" (layer "F.Cu") (at 11.557 178.435)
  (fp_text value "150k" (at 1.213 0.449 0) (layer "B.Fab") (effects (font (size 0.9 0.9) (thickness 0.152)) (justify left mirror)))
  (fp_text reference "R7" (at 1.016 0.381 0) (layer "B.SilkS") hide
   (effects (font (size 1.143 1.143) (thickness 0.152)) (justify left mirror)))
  (pad 1 thru_hole circle (at 3.81 0 0) (size 1.88 1.88) (layers "*.Cu" "*.Paste" "*.Mask") (drill 0.899) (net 5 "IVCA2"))
  (pad 2 thru_hole circle (at -3.81 0 0) (size 1.88 1.88) (layers "*.Cu" "*.Paste" "*.Mask") (drill 0.899) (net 25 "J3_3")))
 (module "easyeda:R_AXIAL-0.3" (layer "F.Cu") (at 11.43 166.497 180)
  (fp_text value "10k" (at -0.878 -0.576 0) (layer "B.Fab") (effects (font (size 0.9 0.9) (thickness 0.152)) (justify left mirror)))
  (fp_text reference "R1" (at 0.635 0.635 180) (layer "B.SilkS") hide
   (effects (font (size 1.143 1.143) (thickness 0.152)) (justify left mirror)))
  (pad 1 thru_hole circle (at 3.81 0 180) (size 1.88 1.88) (layers "*.Cu" "*.Paste" "*.Mask") (drill 0.899) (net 26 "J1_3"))
  (pad 2 thru_hole circle (at -3.81 0 180) (size 1.88 1.88) (layers "*.Cu" "*.Paste" "*.Mask") (drill 0.899) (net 16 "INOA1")))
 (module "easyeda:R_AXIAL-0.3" (layer "F.Cu") (at 12.065 131.572 180)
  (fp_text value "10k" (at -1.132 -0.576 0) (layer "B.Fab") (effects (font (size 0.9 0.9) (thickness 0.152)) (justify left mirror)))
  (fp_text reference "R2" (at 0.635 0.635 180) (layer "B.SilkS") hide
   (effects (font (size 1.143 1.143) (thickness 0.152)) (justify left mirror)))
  (pad 1 thru_hole circle (at 3.81 0 180) (size 1.88 1.88) (layers "*.Cu" "*.Paste" "*.Mask") (drill 0.899) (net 27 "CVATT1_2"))
  (pad 2 thru_hole circle (at -3.81 0 180) (size 1.88 1.88) (layers "*.Cu" "*.Paste" "*.Mask") (drill 0.899) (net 16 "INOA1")))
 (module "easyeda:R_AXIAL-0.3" (layer "F.Cu") (at 11.43 111.252 180)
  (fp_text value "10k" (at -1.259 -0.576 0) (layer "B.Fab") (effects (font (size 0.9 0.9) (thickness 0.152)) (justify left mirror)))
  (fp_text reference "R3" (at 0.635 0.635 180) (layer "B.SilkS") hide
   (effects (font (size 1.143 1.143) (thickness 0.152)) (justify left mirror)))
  (pad 1 thru_hole circle (at 3.81 0 180) (size 1.88 1.88) (layers "*.Cu" "*.Paste" "*.Mask") (drill 0.899) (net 9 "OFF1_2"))
  (pad 2 thru_hole circle (at -3.81 0 180) (size 1.88 1.88) (layers "*.Cu" "*.Paste" "*.Mask") (drill 0.899) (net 16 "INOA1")))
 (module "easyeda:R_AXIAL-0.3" (layer "F.Cu") (at 12.065 134.747 180)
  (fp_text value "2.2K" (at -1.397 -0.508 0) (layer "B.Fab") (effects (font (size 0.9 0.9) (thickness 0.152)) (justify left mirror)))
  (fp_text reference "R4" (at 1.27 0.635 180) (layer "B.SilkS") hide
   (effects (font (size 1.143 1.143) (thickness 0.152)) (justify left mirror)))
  (pad 1 thru_hole circle (at 3.81 0 180) (size 1.88 1.88) (layers "*.Cu" "*.Paste" "*.Mask") (drill 0.899) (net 1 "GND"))
  (pad 2 thru_hole circle (at -3.81 0 180) (size 1.88 1.88) (layers "*.Cu" "*.Paste" "*.Mask") (drill 0.899) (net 13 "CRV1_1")))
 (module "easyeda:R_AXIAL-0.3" (layer "F.Cu") (at 11.557 189.865 180)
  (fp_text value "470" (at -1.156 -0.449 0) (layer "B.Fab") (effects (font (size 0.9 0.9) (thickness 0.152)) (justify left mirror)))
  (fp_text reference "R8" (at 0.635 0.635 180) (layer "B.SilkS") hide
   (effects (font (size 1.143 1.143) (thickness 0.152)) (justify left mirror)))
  (pad 1 thru_hole circle (at 3.81 0 180) (size 1.88 1.88) (layers "*.Cu" "*.Paste" "*.Mask") (drill 0.899) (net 24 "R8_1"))
  (pad 2 thru_hole circle (at -3.81 0 180) (size 1.88 1.88) (layers "*.Cu" "*.Paste" "*.Mask") (drill 0.899) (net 20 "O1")))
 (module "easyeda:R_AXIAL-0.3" (layer "F.Cu") (at 26.67 166.497)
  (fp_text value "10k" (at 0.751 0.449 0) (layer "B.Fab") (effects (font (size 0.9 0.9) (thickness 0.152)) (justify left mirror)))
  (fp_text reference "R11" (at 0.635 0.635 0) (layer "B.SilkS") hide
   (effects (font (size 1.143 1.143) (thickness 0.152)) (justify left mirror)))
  (pad 1 thru_hole circle (at 3.81 0 0) (size 1.88 1.88) (layers "*.Cu" "*.Paste" "*.Mask") (drill 0.899) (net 23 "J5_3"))
  (pad 2 thru_hole circle (at -3.81 0 0) (size 1.88 1.88) (layers "*.Cu" "*.Paste" "*.Mask") (drill 0.899) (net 4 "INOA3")))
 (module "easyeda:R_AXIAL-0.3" (layer "F.Cu") (at 26.67 131.572)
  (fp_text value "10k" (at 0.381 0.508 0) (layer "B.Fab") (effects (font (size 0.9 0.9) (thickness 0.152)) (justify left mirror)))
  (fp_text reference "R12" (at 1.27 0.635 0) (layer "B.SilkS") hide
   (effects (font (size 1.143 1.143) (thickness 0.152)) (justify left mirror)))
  (pad 1 thru_hole circle (at 3.81 0 0) (size 1.88 1.88) (layers "*.Cu" "*.Paste" "*.Mask") (drill 0.899) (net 14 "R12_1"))
  (pad 2 thru_hole circle (at -3.81 0 0) (size 1.88 1.88) (layers "*.Cu" "*.Paste" "*.Mask") (drill 0.899) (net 4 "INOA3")))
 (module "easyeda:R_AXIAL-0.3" (layer "F.Cu") (at 26.035 111.252)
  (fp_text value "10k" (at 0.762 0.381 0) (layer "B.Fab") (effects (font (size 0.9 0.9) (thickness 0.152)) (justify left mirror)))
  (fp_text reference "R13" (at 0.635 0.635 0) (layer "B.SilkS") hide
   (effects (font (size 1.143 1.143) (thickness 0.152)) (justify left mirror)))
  (pad 1 thru_hole circle (at 3.81 0 0) (size 1.88 1.88) (layers "*.Cu" "*.Paste" "*.Mask") (drill 0.899) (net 15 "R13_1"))
  (pad 2 thru_hole circle (at -3.81 0 0) (size 1.88 1.88) (layers "*.Cu" "*.Paste" "*.Mask") (drill 0.899) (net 4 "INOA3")))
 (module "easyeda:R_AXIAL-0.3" (layer "F.Cu") (at 26.67 134.747)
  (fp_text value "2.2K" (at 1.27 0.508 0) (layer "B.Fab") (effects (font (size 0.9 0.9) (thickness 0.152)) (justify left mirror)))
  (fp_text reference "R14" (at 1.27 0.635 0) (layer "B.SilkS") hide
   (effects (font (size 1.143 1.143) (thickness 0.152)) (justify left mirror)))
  (pad 1 thru_hole circle (at 3.81 0 0) (size 1.88 1.88) (layers "*.Cu" "*.Paste" "*.Mask") (drill 0.899) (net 1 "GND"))
  (pad 2 thru_hole circle (at -3.81 0 0) (size 1.88 1.88) (layers "*.Cu" "*.Paste" "*.Mask") (drill 0.899) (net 12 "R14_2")))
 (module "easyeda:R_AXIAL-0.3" (layer "F.Cu") (at 26.797 178.308 180)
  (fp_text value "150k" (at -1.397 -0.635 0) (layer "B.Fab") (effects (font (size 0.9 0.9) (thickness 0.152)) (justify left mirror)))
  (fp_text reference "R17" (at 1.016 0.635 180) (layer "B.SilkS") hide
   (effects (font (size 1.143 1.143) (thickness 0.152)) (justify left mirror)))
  (pad 1 thru_hole circle (at 3.81 0 180) (size 1.88 1.88) (layers "*.Cu" "*.Paste" "*.Mask") (drill 0.899) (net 19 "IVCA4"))
  (pad 2 thru_hole circle (at -3.81 0 180) (size 1.88 1.88) (layers "*.Cu" "*.Paste" "*.Mask") (drill 0.899) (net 22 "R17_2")))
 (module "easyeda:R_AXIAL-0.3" (layer "F.Cu") (at 26.67 189.992)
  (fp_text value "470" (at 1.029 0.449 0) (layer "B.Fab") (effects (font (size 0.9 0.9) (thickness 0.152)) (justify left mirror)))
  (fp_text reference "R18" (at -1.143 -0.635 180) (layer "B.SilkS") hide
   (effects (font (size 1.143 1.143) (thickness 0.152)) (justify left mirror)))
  (pad 1 thru_hole circle (at 3.81 0 0) (size 1.88 1.88) (layers "*.Cu" "*.Paste" "*.Mask") (drill 0.899) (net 21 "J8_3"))
  (pad 2 thru_hole circle (at -3.81 0 0) (size 1.88 1.88) (layers "*.Cu" "*.Paste" "*.Mask") (drill 0.899) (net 3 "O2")))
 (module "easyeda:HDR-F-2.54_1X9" (layer "F.Cu") (at 19.08 153.162 180)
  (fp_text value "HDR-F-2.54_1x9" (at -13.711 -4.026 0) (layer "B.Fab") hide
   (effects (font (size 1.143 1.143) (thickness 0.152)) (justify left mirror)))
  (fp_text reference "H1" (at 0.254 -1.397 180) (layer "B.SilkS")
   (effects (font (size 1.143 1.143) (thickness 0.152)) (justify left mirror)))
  (pad 9 thru_hole circle (at -10.16 0 180) (size 1.575 1.575) (layers "*.Cu" "*.Paste" "*.Mask") (drill 0.889) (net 17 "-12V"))
  (pad 8 thru_hole circle (at -7.62 0 180) (size 1.575 1.575) (layers "*.Cu" "*.Paste" "*.Mask") (drill 0.889) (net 3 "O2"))
  (pad 7 thru_hole circle (at -5.08 0 180) (size 1.575 1.575) (layers "*.Cu" "*.Paste" "*.Mask") (drill 0.889) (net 19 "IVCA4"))
  (pad 6 thru_hole circle (at -2.54 0 180) (size 1.575 1.575) (layers "*.Cu" "*.Paste" "*.Mask") (drill 0.889) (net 4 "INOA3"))
  (pad 5 thru_hole circle (at 0 0 180) (size 1.575 1.575) (layers "*.Cu" "*.Paste" "*.Mask") (drill 0.889) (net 1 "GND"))
  (pad 4 thru_hole circle (at 2.54 0 180) (size 1.575 1.575) (layers "*.Cu" "*.Paste" "*.Mask") (drill 0.889) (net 20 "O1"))
  (pad 3 thru_hole circle (at 5.08 0 180) (size 1.575 1.575) (layers "*.Cu" "*.Paste" "*.Mask") (drill 0.889) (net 5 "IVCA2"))
  (pad 2 thru_hole circle (at 7.62 0 180) (size 1.575 1.575) (layers "*.Cu" "*.Paste" "*.Mask") (drill 0.889) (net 16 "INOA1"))
  (pad 1 thru_hole rect (at 10.16 0 180) (size 1.575 1.575) (layers "*.Cu" "*.Paste" "*.Mask") (drill 0.889) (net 8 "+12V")))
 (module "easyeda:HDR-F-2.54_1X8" (layer "F.Cu") (at 17.81 93.472 180)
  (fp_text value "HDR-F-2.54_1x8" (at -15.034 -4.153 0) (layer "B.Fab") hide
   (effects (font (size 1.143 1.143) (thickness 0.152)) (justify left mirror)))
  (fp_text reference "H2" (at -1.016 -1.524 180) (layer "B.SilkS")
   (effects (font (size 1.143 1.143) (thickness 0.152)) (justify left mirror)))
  (pad 1 thru_hole rect (at 7.62 0 180) (size 1.575 1.575) (layers "*.Cu" "*.Paste" "*.Mask") (drill 0.889) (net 8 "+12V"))
  (pad 2 thru_hole circle (at 5.08 0 180) (size 1.575 1.575) (layers "*.Cu" "*.Paste" "*.Mask") (drill 0.889) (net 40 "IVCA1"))
  (pad 3 thru_hole circle (at 2.54 0 180) (size 1.575 1.575) (layers "*.Cu" "*.Paste" "*.Mask") (drill 0.889) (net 2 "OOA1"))
  (pad 4 thru_hole circle (at 0 0 180) (size 1.575 1.575) (layers "*.Cu" "*.Paste" "*.Mask") (drill 0.889) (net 18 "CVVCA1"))
  (pad 5 thru_hole circle (at -2.54 0 180) (size 1.575 1.575) (layers "*.Cu" "*.Paste" "*.Mask") (drill 0.889) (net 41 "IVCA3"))
  (pad 6 thru_hole circle (at -5.08 0 180) (size 1.575 1.575) (layers "*.Cu" "*.Paste" "*.Mask") (drill 0.889) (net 11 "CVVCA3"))
  (pad 7 thru_hole circle (at -7.62 0 180) (size 1.575 1.575) (layers "*.Cu" "*.Paste" "*.Mask") (drill 0.889) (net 10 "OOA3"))
  (pad 8 thru_hole circle (at -10.16 0 180) (size 1.575 1.575) (layers "*.Cu" "*.Paste" "*.Mask") (drill 0.889) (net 17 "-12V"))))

